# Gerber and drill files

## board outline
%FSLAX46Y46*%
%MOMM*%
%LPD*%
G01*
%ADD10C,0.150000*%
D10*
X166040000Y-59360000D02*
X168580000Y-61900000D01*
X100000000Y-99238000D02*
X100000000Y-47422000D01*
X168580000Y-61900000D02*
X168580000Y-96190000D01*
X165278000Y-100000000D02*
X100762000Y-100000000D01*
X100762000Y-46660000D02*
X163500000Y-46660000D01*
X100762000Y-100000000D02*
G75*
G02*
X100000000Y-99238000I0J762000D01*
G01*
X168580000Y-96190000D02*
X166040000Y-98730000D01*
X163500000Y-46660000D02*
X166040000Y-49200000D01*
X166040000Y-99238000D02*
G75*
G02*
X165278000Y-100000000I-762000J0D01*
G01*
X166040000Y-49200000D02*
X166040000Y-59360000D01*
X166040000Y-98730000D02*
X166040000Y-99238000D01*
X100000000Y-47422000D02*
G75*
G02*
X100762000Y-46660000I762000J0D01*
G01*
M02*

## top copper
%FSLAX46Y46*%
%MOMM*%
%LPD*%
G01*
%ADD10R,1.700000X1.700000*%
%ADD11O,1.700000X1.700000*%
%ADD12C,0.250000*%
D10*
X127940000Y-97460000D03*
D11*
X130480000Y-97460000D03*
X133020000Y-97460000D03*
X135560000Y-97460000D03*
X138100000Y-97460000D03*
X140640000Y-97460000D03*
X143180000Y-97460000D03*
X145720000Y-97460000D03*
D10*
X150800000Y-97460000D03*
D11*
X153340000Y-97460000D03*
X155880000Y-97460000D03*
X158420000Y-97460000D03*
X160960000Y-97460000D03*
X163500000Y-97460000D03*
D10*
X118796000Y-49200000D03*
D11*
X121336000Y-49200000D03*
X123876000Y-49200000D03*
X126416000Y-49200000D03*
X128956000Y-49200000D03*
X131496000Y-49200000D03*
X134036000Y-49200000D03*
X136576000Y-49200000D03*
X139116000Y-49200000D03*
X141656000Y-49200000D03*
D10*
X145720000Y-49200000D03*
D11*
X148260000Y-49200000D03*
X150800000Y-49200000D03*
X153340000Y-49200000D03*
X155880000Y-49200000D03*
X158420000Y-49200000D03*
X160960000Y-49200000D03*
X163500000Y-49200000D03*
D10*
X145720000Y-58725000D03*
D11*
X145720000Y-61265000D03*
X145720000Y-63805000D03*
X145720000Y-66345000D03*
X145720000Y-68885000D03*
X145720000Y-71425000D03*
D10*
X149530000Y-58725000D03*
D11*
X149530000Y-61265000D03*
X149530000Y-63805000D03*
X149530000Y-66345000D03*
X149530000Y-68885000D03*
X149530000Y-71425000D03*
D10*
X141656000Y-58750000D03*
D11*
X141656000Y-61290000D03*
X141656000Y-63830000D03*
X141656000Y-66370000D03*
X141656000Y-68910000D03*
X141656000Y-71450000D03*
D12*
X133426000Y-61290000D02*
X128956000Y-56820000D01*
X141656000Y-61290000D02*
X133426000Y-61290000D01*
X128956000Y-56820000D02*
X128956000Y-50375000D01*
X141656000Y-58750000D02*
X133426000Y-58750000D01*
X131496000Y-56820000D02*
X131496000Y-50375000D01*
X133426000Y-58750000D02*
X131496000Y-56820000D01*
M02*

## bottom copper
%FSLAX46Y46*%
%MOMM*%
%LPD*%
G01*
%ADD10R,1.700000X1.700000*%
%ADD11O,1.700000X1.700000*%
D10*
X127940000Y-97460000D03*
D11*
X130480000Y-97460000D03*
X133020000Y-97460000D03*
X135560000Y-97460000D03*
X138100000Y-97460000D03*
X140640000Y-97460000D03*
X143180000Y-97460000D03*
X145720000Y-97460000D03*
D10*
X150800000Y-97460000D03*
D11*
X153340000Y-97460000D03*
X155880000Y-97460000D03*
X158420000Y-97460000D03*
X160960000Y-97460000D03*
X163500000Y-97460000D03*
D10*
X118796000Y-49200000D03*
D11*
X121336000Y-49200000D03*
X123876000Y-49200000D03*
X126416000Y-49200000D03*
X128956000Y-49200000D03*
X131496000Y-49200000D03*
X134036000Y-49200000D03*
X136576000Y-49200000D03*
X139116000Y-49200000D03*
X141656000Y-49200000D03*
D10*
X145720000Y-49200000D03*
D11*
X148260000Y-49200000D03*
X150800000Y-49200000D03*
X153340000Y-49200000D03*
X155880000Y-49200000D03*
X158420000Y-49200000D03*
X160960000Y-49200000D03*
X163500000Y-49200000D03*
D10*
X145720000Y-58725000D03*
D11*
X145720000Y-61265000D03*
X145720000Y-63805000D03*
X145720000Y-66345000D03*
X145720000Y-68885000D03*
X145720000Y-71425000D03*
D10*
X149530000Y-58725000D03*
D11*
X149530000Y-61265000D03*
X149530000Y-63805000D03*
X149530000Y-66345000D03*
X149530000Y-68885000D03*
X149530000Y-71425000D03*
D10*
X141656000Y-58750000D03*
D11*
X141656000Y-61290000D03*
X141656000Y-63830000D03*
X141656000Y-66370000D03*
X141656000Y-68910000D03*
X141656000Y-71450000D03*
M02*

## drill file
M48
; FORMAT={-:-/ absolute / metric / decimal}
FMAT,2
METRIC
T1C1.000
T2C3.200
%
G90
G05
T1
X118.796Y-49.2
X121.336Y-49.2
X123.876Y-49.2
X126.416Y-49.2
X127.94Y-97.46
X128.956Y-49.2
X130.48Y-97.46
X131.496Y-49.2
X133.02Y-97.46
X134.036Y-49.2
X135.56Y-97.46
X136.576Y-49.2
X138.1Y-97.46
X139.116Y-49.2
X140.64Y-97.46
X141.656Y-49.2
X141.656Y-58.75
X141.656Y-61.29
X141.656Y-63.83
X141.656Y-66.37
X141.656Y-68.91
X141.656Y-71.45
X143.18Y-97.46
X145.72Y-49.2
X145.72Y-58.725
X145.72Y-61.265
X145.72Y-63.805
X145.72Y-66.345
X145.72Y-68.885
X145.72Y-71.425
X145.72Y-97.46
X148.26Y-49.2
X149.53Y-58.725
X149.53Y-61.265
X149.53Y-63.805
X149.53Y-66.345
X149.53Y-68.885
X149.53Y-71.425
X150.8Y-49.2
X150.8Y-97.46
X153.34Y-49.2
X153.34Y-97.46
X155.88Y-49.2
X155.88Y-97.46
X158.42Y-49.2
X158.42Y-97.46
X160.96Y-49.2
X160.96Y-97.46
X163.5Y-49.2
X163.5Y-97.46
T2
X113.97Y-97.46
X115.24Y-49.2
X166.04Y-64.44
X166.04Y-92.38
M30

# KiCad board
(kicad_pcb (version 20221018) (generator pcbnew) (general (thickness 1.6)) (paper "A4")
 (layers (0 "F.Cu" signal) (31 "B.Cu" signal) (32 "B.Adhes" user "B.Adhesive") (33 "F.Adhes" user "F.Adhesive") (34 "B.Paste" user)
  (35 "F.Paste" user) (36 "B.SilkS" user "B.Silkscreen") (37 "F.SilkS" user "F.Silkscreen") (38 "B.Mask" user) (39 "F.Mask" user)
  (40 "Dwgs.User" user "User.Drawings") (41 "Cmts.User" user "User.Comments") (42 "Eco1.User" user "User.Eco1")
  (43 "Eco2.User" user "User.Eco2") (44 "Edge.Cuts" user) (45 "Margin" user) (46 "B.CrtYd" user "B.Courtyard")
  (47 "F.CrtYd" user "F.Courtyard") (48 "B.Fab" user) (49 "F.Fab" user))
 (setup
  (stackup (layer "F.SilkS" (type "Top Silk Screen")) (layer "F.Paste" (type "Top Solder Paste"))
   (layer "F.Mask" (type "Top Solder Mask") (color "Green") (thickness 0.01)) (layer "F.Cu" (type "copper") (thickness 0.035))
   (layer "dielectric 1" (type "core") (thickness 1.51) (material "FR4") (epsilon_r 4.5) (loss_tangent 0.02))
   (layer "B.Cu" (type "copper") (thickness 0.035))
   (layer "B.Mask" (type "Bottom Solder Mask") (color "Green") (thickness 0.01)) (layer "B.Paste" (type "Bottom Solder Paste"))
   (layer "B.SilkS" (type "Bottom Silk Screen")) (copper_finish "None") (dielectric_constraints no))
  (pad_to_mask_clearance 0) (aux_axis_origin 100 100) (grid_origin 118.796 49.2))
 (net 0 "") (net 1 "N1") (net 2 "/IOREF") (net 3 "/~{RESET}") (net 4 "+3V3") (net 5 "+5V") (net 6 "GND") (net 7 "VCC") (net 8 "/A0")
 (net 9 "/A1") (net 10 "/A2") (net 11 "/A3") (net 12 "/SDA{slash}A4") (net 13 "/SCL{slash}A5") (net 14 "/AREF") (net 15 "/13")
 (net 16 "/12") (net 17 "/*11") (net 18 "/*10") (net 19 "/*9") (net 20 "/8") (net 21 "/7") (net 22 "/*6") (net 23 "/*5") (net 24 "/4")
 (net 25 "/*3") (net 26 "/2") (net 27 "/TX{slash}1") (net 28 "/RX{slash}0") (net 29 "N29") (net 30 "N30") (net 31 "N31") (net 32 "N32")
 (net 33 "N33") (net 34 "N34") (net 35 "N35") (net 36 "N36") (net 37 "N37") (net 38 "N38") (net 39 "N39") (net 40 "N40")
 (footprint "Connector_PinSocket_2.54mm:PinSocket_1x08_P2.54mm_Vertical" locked (layer "F.Cu") (at 127.94 97.46 90)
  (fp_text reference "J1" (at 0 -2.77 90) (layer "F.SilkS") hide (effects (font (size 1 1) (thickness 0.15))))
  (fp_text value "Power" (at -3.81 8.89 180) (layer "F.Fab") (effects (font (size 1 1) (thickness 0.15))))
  (pad "1" thru_hole rect locked (at 0 0 90) (size 1.7 1.7) (drill 1) (layers "*.Cu" "*.Mask") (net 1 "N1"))
  (pad "2" thru_hole oval locked (at 0 2.54 90) (size 1.7 1.7) (drill 1) (layers "*.Cu" "*.Mask") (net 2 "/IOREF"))
  (pad "3" thru_hole oval locked (at 0 5.08 90) (size 1.7 1.7) (drill 1) (layers "*.Cu" "*.Mask") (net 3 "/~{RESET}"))
  (pad "4" thru_hole oval locked (at 0 7.62 90) (size 1.7 1.7) (drill 1) (layers "*.Cu" "*.Mask") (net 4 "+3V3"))
  (pad "5" thru_hole oval locked (at 0 10.16 90) (size 1.7 1.7) (drill 1) (layers "*.Cu" "*.Mask") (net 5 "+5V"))
  (pad "6" thru_hole oval locked (at 0 12.7 90) (size 1.7 1.7) (drill 1) (layers "*.Cu" "*.Mask") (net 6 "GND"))
  (pad "7" thru_hole oval locked (at 0 15.24 90) (size 1.7 1.7) (drill 1) (layers "*.Cu" "*.Mask") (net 6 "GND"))
  (pad "8" thru_hole oval locked (at 0 17.78 90) (size 1.7 1.7) (drill 1) (layers "*.Cu" "*.Mask") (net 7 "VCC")))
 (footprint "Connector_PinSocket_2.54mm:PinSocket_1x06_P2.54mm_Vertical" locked (layer "F.Cu") (at 150.8 97.46 90)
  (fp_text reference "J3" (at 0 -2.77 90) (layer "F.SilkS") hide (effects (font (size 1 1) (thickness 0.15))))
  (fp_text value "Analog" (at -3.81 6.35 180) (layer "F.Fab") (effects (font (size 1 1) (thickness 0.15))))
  (pad "1" thru_hole rect locked (at 0 0 90) (size 1.7 1.7) (drill 1) (layers "*.Cu" "*.Mask") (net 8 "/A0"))
  (pad "2" thru_hole oval locked (at 0 2.54 90) (size 1.7 1.7) (drill 1) (layers "*.Cu" "*.Mask") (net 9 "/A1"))
  (pad "3" thru_hole oval locked (at 0 5.08 90) (size 1.7 1.7) (drill 1) (layers "*.Cu" "*.Mask") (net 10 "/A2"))
  (pad "4" thru_hole oval locked (at 0 7.62 90) (size 1.7 1.7) (drill 1) (layers "*.Cu" "*.Mask") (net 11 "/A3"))
  (pad "5" thru_hole oval locked (at 0 10.16 90) (size 1.7 1.7) (drill 1) (layers "*.Cu" "*.Mask") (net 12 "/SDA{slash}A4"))
  (pad "6" thru_hole oval locked (at 0 12.7 90) (size 1.7 1.7) (drill 1) (layers "*.Cu" "*.Mask") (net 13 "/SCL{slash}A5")))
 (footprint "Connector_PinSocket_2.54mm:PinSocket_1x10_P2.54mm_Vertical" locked (layer "F.Cu") (at 118.796 49.2 90)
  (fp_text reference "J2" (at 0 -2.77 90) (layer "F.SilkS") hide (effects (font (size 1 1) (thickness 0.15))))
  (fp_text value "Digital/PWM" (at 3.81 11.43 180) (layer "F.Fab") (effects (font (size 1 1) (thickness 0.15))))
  (pad "1" thru_hole rect locked (at 0 0 90) (size 1.7 1.7) (drill 1) (layers "*.Cu" "*.Mask") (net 13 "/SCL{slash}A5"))
  (pad "2" thru_hole oval locked (at 0 2.54 90) (size 1.7 1.7) (drill 1) (layers "*.Cu" "*.Mask") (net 12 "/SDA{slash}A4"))
  (pad "3" thru_hole oval locked (at 0 5.08 90) (size 1.7 1.7) (drill 1) (layers "*.Cu" "*.Mask") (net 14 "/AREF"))
  (pad "4" thru_hole oval locked (at 0 7.62 90) (size 1.7 1.7) (drill 1) (layers "*.Cu" "*.Mask") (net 6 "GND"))
  (pad "5" thru_hole oval locked (at 0 10.16 90) (size 1.7 1.7) (drill 1) (layers "*.Cu" "*.Mask") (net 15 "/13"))
  (pad "6" thru_hole oval locked (at 0 12.7 90) (size 1.7 1.7) (drill 1) (layers "*.Cu" "*.Mask") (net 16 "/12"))
  (pad "7" thru_hole oval locked (at 0 15.24 90) (size 1.7 1.7) (drill 1) (layers "*.Cu" "*.Mask") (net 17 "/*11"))
  (pad "8" thru_hole oval locked (at 0 17.78 90) (size 1.7 1.7) (drill 1) (layers "*.Cu" "*.Mask") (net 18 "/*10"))
  (pad "9" thru_hole oval locked (at 0 20.32 90) (size 1.7 1.7) (drill 1) (layers "*.Cu" "*.Mask") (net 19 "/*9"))
  (pad "10" thru_hole oval locked (at 0 22.86 90) (size 1.7 1.7) (drill 1) (layers "*.Cu" "*.Mask") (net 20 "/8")))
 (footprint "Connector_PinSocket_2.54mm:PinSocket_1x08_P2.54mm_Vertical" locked (layer "F.Cu") (at 145.72 49.2 90)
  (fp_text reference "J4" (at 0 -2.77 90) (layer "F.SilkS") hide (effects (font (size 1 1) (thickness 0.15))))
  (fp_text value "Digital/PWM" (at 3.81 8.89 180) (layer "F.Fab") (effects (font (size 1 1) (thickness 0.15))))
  (pad "1" thru_hole rect locked (at 0 0 90) (size 1.7 1.7) (drill 1) (layers "*.Cu" "*.Mask") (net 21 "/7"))
  (pad "2" thru_hole oval locked (at 0 2.54 90) (size 1.7 1.7) (drill 1) (layers "*.Cu" "*.Mask") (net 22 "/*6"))
  (pad "3" thru_hole oval locked (at 0 5.08 90) (size 1.7 1.7) (drill 1) (layers "*.Cu" "*.Mask") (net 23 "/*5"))
  (pad "4" thru_hole oval locked (at 0 7.62 90) (size 1.7 1.7) (drill 1) (layers "*.Cu" "*.Mask") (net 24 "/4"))
  (pad "5" thru_hole oval locked (at 0 10.16 90) (size 1.7 1.7) (drill 1) (layers "*.Cu" "*.Mask") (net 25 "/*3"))
  (pad "6" thru_hole oval locked (at 0 12.7 90) (size 1.7 1.7) (drill 1) (layers "*.Cu" "*.Mask") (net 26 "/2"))
  (pad "7" thru_hole oval locked (at 0 15.24 90) (size 1.7 1.7) (drill 1) (layers "*.Cu" "*.Mask") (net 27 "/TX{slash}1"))
  (pad "8" thru_hole oval locked (at 0 17.78 90) (size 1.7 1.7) (drill 1) (layers "*.Cu" "*.Mask") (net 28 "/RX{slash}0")))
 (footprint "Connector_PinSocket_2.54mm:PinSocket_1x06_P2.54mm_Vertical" (layer "F.Cu") (at 145.72 58.725)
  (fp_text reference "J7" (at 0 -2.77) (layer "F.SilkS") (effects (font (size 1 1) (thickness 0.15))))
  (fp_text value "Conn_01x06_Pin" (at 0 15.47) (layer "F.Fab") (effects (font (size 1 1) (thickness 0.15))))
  (pad "1" thru_hole rect (at 0 0) (size 1.7 1.7) (drill 1) (layers "*.Cu" "*.Mask") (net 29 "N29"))
  (pad "2" thru_hole oval (at 0 2.54) (size 1.7 1.7) (drill 1) (layers "*.Cu" "*.Mask") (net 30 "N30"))
  (pad "3" thru_hole oval (at 0 5.08) (size 1.7 1.7) (drill 1) (layers "*.Cu" "*.Mask") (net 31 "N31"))
  (pad "4" thru_hole oval (at 0 7.62) (size 1.7 1.7) (drill 1) (layers "*.Cu" "*.Mask") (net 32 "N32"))
  (pad "5" thru_hole oval (at 0 10.16) (size 1.7 1.7) (drill 1) (layers "*.Cu" "*.Mask") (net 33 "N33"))
  (pad "6" thru_hole oval (at 0 12.7) (size 1.7 1.7) (drill 1) (layers "*.Cu" "*.Mask") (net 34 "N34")))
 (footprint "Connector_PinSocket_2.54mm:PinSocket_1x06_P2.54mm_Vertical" (layer "F.Cu") (at 149.53 58.725)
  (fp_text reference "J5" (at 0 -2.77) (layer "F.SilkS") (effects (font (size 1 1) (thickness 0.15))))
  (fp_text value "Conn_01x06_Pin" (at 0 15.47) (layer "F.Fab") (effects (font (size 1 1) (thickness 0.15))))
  (pad "1" thru_hole rect (at 0 0) (size 1.7 1.7) (drill 1) (layers "*.Cu" "*.Mask") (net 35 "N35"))
  (pad "2" thru_hole oval (at 0 2.54) (size 1.7 1.7) (drill 1) (layers "*.Cu" "*.Mask") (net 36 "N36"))
  (pad "3" thru_hole oval (at 0 5.08) (size 1.7 1.7) (drill 1) (layers "*.Cu" "*.Mask") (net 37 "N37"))
  (pad "4" thru_hole oval (at 0 7.62) (size 1.7 1.7) (drill 1) (layers "*.Cu" "*.Mask") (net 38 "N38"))
  (pad "5" thru_hole oval (at 0 10.16) (size 1.7 1.7) (drill 1) (layers "*.Cu" "*.Mask") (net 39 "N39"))
  (pad "6" thru_hole oval (at 0 12.7) (size 1.7 1.7) (drill 1) (layers "*.Cu" "*.Mask") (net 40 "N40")))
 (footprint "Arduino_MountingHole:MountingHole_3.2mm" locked (layer "F.Cu") (at 115.24 49.2)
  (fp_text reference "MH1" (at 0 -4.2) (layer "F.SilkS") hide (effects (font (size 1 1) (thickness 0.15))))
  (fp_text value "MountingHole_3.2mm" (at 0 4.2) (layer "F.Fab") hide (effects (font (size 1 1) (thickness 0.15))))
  (pad "" np_thru_hole circle locked (at 0 0) (size 3.2 3.2) (drill 3.2) (layers "*.Cu" "*.Mask")))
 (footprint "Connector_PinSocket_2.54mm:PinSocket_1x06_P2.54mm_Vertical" (layer "F.Cu") (at 141.656 58.75)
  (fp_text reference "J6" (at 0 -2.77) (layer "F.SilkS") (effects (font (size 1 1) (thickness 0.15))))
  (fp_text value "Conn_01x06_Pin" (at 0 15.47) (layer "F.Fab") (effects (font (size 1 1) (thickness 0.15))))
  (pad "1" thru_hole rect (at 0 0) (size 1.7 1.7) (drill 1) (layers "*.Cu" "*.Mask") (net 16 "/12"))
  (pad "2" thru_hole oval (at 0 2.54) (size 1.7 1.7) (drill 1) (layers "*.Cu" "*.Mask") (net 15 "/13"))
  (pad "3" thru_hole oval (at 0 5.08) (size 1.7 1.7) (drill 1) (layers "*.Cu" "*.Mask") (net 20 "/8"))
  (pad "4" thru_hole oval (at 0 7.62) (size 1.7 1.7) (drill 1) (layers "*.Cu" "*.Mask") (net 21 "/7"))
  (pad "5" thru_hole oval (at 0 10.16) (size 1.7 1.7) (drill 1) (layers "*.Cu" "*.Mask") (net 24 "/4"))
  (pad "6" thru_hole oval (at 0 12.7) (size 1.7 1.7) (drill 1) (layers "*.Cu" "*.Mask") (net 26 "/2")))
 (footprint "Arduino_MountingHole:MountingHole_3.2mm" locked (layer "F.Cu") (at 113.97 97.46)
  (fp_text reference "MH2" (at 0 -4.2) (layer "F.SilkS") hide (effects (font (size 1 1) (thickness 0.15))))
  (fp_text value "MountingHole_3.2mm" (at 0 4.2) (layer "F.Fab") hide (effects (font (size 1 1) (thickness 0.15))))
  (pad "" np_thru_hole circle locked (at 0 0) (size 3.2 3.2) (drill 3.2) (layers "*.Cu" "*.Mask")))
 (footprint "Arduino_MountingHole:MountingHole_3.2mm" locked (layer "F.Cu") (at 166.04 64.44)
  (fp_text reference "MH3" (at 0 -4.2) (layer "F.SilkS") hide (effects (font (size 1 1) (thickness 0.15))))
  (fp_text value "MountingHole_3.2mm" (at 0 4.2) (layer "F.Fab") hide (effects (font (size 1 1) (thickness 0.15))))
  (pad "" np_thru_hole circle locked (at 0 0) (size 3.2 3.2) (drill 3.2) (layers "*.Cu" "*.Mask")))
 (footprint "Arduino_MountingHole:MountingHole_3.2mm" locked (layer "F.Cu") (at 166.04 92.38)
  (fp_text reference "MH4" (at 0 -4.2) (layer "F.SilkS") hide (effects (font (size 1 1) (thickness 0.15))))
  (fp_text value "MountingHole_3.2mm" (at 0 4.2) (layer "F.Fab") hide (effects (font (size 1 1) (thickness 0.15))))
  (pad "" np_thru_hole circle locked (at 0 0) (size 3.2 3.2) (drill 3.2) (layers "*.Cu" "*.Mask")))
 (gr_line (start 166.04 59.36) (end 168.58 61.9) (stroke (width 0.15) (type solid)) (layer "Edge.Cuts"))
 (gr_line (start 100 99.238) (end 100 47.422) (stroke (width 0.15) (type solid)) (layer "Edge.Cuts"))
 (gr_line (start 168.58 61.9) (end 168.58 96.19) (stroke (width 0.15) (type solid)) (layer "Edge.Cuts"))
 (gr_line (start 165.278 100) (end 100.762 100) (stroke (width 0.15) (type solid)) (layer "Edge.Cuts"))
 (gr_line (start 100.762 46.66) (end 163.5 46.66) (stroke (width 0.15) (type solid)) (layer "Edge.Cuts"))
 (gr_arc (start 100.762 100) (mid 100.223185 99.776815) (end 100 99.238) (stroke (width 0.15) (type solid)) (layer "Edge.Cuts"))
 (gr_line (start 168.58 96.19) (end 166.04 98.73) (stroke (width 0.15) (type solid)) (layer "Edge.Cuts"))
 (gr_line (start 163.5 46.66) (end 166.04 49.2) (stroke (width 0.15) (type solid)) (layer "Edge.Cuts"))
 (gr_arc (start 166.04 99.238) (mid 165.816815 99.776815) (end 165.278 100) (stroke (width 0.15) (type solid)) (layer "Edge.Cuts"))
 (gr_line (start 166.04 49.2) (end 166.04 59.36) (stroke (width 0.15) (type solid)) (layer "Edge.Cuts"))
 (gr_line (start 166.04 98.73) (end 166.04 99.238) (stroke (width 0.15) (type solid)) (layer "Edge.Cuts"))
 (gr_arc (start 100 47.422) (mid 100.223185 46.883185) (end 100.762 46.66) (stroke (width 0.15) (type solid)) (layer "Edge.Cuts"))
 (segment (start 133.426 61.29) (end 128.956 56.82) (width 0.25) (layer "F.Cu") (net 15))
 (segment (start 141.656 61.29) (end 133.426 61.29) (width 0.25) (layer "F.Cu") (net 15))
 (segment (start 128.956 56.82) (end 128.956 50.375) (width 0.25) (layer "F.Cu") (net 15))
 (segment (start 141.656 58.75) (end 133.426 58.75) (width 0.25) (layer "F.Cu") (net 16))
 (segment (start 131.496 56.82) (end 131.496 50.375) (width 0.25) (layer "F.Cu") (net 16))
 (segment (start 133.426 58.75) (end 131.496 56.82) (width 0.25) (layer "F.Cu") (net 16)))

